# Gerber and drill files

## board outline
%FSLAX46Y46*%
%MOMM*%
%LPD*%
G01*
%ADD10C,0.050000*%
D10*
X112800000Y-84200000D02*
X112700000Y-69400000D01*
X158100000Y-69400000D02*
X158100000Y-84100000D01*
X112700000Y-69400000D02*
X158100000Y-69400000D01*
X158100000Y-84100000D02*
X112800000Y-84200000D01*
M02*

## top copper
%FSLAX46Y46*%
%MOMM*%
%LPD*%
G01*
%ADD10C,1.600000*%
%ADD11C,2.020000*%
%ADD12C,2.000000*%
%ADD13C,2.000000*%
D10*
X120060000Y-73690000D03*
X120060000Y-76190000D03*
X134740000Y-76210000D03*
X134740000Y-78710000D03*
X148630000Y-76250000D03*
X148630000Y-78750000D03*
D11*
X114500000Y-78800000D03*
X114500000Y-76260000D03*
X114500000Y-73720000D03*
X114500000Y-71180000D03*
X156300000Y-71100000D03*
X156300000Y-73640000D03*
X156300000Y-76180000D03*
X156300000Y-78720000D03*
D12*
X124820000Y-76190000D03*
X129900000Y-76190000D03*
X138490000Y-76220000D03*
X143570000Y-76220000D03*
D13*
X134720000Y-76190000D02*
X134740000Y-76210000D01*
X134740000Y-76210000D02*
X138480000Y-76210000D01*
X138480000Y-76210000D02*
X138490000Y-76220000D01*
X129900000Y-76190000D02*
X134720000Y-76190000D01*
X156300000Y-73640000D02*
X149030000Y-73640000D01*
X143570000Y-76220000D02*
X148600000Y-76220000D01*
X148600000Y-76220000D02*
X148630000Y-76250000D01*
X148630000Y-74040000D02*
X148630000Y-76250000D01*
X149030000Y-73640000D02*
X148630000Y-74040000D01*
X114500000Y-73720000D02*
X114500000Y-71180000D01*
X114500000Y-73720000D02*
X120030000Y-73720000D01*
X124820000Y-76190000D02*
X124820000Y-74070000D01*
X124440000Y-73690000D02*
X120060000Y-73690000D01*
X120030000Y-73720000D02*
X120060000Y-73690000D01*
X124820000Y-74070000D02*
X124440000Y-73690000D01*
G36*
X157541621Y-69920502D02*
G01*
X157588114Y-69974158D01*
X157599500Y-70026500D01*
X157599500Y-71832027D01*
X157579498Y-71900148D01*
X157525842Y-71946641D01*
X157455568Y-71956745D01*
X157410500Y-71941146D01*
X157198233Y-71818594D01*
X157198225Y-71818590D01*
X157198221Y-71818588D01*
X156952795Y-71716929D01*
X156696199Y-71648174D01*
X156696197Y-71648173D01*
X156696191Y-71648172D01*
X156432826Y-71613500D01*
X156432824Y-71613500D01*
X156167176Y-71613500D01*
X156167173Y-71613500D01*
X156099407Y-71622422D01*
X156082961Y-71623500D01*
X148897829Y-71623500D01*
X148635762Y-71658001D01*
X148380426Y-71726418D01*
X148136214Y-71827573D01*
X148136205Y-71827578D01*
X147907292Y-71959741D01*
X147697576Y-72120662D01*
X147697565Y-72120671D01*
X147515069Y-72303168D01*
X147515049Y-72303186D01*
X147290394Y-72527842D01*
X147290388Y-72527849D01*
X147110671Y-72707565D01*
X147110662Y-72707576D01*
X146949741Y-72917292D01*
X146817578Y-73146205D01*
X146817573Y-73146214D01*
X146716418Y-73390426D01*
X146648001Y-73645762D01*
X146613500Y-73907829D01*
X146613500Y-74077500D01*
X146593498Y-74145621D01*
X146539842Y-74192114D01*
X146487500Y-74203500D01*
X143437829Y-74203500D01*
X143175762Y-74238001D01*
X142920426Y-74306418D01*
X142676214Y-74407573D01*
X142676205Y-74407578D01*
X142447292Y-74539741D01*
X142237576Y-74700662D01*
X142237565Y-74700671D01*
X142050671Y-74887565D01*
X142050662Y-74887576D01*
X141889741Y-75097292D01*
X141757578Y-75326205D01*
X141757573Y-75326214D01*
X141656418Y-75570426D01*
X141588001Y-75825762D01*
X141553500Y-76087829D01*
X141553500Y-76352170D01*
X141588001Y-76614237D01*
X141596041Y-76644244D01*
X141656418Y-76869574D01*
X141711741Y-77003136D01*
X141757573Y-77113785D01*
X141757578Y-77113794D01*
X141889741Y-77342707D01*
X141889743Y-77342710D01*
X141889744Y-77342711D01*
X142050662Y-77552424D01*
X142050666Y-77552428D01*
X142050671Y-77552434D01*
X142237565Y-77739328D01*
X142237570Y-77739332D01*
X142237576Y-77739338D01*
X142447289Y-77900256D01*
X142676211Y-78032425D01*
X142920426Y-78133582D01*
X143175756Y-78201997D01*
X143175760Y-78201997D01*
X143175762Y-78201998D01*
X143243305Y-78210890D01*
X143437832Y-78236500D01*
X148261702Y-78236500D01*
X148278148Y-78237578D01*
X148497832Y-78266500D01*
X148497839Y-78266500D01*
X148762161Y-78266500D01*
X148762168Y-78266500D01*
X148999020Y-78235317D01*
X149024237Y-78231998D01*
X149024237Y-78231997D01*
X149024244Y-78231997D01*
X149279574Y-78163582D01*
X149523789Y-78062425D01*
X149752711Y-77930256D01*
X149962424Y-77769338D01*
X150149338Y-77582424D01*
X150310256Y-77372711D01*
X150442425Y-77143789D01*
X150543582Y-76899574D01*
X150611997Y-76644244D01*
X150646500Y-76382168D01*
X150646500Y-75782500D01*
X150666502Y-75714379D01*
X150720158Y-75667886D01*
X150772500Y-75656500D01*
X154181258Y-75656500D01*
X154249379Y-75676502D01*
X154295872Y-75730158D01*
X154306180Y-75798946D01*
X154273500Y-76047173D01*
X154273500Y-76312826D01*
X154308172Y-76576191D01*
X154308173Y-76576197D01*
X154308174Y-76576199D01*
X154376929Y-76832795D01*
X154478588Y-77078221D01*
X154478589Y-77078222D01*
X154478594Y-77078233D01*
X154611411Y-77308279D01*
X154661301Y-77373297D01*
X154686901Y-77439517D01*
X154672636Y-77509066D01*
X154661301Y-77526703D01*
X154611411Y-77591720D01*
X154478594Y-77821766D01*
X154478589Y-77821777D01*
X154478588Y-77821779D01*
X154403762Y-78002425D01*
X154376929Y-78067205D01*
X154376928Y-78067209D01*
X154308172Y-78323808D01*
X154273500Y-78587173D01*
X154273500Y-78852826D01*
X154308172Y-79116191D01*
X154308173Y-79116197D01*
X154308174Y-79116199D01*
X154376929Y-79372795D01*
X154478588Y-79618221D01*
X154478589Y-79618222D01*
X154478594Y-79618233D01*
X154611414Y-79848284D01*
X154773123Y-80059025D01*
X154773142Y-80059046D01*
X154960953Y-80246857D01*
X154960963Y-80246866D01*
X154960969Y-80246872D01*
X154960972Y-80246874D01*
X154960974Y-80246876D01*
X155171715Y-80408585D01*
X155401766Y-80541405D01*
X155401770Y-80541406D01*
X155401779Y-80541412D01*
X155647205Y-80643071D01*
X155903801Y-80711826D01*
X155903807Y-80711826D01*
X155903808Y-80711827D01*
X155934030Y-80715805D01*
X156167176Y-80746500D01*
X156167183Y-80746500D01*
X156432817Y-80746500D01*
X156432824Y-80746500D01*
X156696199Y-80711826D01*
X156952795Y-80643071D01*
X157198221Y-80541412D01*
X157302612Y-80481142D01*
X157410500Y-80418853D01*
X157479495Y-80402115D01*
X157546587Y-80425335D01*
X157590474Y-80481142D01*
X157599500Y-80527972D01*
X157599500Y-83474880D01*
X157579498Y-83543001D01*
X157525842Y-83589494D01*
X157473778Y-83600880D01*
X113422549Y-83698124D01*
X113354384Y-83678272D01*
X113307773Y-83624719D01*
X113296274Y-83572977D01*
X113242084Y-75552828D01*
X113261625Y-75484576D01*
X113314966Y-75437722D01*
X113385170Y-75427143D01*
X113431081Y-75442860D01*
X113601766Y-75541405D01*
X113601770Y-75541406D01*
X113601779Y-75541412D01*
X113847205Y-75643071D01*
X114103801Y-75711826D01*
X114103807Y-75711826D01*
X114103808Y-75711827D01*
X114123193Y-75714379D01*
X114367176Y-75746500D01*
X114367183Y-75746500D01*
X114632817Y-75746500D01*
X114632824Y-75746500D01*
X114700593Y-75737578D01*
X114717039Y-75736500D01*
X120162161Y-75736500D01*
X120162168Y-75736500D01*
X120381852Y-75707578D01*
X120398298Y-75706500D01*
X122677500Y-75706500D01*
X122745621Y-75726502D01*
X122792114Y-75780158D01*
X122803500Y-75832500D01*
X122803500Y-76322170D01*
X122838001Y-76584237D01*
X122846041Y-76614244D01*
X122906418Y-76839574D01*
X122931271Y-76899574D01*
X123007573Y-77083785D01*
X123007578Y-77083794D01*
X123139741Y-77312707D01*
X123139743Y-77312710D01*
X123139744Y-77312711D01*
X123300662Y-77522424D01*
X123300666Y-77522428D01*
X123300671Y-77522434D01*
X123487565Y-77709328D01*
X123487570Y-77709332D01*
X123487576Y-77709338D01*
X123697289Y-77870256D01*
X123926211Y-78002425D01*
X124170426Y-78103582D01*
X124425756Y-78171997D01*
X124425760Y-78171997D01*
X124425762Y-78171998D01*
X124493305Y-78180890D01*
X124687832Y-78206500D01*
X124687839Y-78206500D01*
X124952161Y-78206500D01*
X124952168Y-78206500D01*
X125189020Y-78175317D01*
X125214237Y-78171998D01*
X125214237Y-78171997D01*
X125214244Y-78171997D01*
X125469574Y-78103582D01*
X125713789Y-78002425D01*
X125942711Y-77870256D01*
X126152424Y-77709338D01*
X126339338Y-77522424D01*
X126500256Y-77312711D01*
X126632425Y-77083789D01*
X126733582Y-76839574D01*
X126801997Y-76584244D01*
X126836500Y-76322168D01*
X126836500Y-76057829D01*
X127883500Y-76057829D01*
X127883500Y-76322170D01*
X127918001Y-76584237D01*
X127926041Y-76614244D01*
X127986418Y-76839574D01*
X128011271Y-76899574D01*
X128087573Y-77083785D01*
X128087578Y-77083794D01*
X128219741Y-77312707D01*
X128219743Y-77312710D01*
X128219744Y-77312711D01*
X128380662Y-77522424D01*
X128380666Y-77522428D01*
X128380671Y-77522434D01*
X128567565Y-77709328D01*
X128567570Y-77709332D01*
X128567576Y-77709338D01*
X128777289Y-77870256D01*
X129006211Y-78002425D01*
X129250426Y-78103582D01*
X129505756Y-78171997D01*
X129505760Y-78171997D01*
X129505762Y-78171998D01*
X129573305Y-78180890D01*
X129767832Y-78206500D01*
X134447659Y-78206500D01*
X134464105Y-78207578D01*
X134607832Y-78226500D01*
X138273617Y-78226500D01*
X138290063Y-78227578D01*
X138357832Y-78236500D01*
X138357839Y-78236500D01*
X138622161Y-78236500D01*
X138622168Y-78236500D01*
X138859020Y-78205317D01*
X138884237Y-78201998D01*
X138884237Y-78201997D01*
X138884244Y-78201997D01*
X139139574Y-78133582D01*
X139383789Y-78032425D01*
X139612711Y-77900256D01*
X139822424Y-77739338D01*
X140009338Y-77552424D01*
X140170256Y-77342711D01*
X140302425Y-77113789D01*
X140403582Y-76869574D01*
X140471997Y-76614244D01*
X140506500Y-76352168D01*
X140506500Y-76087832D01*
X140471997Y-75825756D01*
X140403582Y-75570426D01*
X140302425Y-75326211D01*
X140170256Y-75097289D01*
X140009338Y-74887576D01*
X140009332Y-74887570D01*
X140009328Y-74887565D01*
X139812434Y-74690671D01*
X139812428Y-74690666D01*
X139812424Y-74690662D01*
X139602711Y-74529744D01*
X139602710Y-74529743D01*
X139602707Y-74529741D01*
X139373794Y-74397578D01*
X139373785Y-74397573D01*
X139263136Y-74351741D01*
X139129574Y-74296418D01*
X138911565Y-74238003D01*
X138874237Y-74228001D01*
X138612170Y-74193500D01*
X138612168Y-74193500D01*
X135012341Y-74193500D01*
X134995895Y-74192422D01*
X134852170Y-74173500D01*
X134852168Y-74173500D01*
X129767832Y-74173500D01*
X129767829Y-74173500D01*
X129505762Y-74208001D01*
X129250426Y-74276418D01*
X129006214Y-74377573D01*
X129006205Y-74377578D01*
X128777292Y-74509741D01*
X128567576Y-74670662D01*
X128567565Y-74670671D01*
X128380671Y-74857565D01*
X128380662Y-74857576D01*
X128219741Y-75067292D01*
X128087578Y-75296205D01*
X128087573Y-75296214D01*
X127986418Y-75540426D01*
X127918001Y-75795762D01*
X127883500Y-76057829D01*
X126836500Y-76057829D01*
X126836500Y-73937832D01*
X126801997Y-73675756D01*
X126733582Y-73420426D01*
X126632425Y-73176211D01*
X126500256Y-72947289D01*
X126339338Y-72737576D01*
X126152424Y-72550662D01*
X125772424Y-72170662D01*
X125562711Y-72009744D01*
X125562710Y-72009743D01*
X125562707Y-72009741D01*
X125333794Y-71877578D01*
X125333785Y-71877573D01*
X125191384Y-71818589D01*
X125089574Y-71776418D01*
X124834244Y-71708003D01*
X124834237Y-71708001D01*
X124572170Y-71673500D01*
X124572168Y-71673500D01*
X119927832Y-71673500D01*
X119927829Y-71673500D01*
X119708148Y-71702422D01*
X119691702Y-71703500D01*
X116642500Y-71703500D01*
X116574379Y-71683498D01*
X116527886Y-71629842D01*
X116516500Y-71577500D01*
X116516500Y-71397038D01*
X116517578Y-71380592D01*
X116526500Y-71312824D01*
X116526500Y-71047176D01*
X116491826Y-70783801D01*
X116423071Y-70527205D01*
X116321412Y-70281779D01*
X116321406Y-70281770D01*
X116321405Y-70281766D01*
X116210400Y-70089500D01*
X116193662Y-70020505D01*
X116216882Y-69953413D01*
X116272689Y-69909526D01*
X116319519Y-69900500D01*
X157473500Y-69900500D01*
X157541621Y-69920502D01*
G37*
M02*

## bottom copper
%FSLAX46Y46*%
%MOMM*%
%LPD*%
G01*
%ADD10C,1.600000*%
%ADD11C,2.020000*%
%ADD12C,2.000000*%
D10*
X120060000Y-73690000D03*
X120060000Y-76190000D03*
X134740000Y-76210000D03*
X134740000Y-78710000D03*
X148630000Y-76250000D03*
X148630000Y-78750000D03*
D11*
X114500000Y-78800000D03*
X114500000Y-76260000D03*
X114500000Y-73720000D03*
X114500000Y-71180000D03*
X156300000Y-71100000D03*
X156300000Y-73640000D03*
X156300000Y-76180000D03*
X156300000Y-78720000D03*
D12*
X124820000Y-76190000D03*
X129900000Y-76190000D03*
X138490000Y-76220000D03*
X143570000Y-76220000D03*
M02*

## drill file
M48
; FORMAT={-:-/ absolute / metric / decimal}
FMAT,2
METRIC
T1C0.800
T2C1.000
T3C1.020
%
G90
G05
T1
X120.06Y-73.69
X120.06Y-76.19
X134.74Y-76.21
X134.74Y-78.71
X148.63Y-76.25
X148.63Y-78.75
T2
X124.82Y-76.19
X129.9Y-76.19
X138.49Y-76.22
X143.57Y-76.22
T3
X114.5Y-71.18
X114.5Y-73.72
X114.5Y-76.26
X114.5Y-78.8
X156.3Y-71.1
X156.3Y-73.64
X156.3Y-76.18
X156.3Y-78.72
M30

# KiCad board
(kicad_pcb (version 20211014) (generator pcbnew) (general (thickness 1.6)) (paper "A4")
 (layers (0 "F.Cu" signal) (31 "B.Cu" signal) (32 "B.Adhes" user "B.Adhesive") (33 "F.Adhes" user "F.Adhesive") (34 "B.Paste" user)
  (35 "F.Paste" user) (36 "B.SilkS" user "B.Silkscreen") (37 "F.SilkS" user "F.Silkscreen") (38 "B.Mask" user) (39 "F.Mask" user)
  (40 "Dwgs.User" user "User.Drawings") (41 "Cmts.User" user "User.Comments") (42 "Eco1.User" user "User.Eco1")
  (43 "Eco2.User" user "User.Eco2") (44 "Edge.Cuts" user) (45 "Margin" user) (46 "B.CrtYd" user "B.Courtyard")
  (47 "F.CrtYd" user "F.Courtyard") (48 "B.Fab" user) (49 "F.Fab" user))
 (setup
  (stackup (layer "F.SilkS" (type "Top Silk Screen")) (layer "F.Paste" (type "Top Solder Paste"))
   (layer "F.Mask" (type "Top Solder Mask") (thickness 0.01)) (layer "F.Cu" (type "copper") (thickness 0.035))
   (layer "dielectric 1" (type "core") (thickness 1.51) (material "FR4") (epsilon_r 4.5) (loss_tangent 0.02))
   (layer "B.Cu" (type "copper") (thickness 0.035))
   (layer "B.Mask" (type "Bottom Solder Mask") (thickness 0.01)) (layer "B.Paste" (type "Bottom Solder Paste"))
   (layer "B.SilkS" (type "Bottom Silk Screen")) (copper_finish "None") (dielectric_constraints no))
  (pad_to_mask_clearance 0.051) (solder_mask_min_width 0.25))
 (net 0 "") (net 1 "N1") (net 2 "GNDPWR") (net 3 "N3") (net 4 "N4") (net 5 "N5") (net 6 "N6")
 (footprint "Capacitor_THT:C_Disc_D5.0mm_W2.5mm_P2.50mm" (layer "F.Cu") (at 120.06 73.69 -90)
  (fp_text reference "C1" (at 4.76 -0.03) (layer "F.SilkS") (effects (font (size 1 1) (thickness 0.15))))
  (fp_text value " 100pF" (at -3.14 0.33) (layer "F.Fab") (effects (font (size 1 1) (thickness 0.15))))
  (pad "1" thru_hole circle locked (at 0 0 270) (size 1.6 1.6) (drill 0.8) (layers *.Cu *.Mask) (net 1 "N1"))
  (pad "2" thru_hole circle locked (at 2.5 0 270) (size 1.6 1.6) (drill 0.8) (layers *.Cu *.Mask) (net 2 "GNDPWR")))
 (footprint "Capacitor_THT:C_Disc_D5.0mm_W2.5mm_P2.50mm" (layer "F.Cu") (at 134.74 76.21 -90)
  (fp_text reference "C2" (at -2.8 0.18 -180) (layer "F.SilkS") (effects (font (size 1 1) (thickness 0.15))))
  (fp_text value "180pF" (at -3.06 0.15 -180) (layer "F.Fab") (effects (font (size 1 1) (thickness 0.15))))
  (pad "1" thru_hole circle locked (at 0 0 270) (size 1.6 1.6) (drill 0.8) (layers *.Cu *.Mask) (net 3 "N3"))
  (pad "2" thru_hole circle locked (at 2.5 0 270) (size 1.6 1.6) (drill 0.8) (layers *.Cu *.Mask) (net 2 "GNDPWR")))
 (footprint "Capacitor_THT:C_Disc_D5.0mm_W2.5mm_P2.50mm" (layer "F.Cu") (at 148.63 76.25 -90)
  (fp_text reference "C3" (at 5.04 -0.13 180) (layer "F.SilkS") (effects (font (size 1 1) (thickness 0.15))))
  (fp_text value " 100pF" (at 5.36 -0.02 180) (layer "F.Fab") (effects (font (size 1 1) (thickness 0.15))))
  (pad "1" thru_hole circle locked (at 0 0 270) (size 1.6 1.6) (drill 0.8) (layers *.Cu *.Mask) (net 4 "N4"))
  (pad "2" thru_hole circle locked (at 2.5 0 270) (size 1.6 1.6) (drill 0.8) (layers *.Cu *.Mask) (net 2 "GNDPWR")))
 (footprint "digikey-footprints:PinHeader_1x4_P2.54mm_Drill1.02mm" (layer "F.Cu") (at 114.5 78.8 90)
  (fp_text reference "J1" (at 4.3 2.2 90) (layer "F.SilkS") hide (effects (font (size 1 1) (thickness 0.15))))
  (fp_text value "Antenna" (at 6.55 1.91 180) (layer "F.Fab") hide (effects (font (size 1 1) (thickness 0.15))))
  (pad "1" thru_hole circle locked (at 0 0 90) (size 2.02 2.02) (drill 1.02) (layers *.Cu *.Mask) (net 2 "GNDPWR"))
  (pad "2" thru_hole circle locked (at 2.54 0 90) (size 2.02 2.02) (drill 1.02) (layers *.Cu *.Mask) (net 2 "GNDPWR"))
  (pad "3" thru_hole circle locked (at 5.08 0 90) (size 2.02 2.02) (drill 1.02) (layers *.Cu *.Mask) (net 1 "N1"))
  (pad "4" thru_hole circle locked (at 7.62 0 90) (size 2.02 2.02) (drill 1.02) (layers *.Cu *.Mask) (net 1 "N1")))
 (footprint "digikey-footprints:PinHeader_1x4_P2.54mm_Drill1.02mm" (layer "F.Cu") (at 156.3 71.1 -90)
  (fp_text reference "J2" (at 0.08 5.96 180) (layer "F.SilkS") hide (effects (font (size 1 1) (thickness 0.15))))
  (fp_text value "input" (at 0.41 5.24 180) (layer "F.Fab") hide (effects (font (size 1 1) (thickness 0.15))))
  (pad "1" thru_hole circle locked (at 0 0 270) (size 2.02 2.02) (drill 1.02) (layers *.Cu *.Mask) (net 2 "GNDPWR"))
  (pad "2" thru_hole circle locked (at 2.54 0 270) (size 2.02 2.02) (drill 1.02) (layers *.Cu *.Mask) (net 4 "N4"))
  (pad "3" thru_hole circle locked (at 5.08 0 270) (size 2.02 2.02) (drill 1.02) (layers *.Cu *.Mask) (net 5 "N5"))
  (pad "4" thru_hole circle locked (at 7.62 0 270) (size 2.02 2.02) (drill 1.02) (layers *.Cu *.Mask) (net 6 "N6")))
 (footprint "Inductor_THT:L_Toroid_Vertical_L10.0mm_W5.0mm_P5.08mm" (layer "F.Cu") (at 124.82 76.19 90)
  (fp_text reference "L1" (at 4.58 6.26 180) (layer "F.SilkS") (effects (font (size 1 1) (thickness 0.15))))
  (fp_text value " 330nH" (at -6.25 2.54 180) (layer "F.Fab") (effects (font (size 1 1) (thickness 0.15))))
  (pad "1" thru_hole circle locked (at 0 0 90) (size 2 2) (drill 1) (layers *.Cu *.Mask) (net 1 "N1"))
  (pad "2" thru_hole circle locked (at 0 5.08 90) (size 2 2) (drill 1) (layers *.Cu *.Mask) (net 3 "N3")))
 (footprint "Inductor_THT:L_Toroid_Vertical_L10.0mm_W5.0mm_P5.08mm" (layer "F.Cu") (at 138.49 76.22 90)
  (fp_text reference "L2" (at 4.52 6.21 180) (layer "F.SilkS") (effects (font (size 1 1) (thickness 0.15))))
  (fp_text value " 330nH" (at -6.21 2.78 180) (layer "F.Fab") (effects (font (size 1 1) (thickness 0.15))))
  (pad "1" thru_hole circle locked (at 0 0 90) (size 2 2) (drill 1) (layers *.Cu *.Mask) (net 3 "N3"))
  (pad "2" thru_hole circle locked (at 0 5.08 90) (size 2 2) (drill 1) (layers *.Cu *.Mask) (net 4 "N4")))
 (gr_line (start 112.8 84.2) (end 112.7 69.4) (layer "Edge.Cuts") (width 0.05))
 (gr_line (start 158.1 69.4) (end 158.1 84.1) (layer "Edge.Cuts") (width 0.05))
 (gr_line (start 112.7 69.4) (end 158.1 69.4) (layer "Edge.Cuts") (width 0.05))
 (gr_line (start 158.1 84.1) (end 112.8 84.2) (layer "Edge.Cuts") (width 0.05))
 (segment (start 134.72 76.19) (end 134.74 76.21) (width 2) (layer "F.Cu") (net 3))
 (segment (start 134.74 76.21) (end 138.48 76.21) (width 2) (layer "F.Cu") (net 3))
 (segment (start 138.48 76.21) (end 138.49 76.22) (width 2) (layer "F.Cu") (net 3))
 (segment (start 129.9 76.19) (end 134.72 76.19) (width 2) (layer "F.Cu") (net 3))
 (segment (start 156.3 73.64) (end 149.03 73.64) (width 2) (layer "F.Cu") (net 4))
 (segment (start 143.57 76.22) (end 148.6 76.22) (width 2) (layer "F.Cu") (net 4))
 (segment (start 148.6 76.22) (end 148.63 76.25) (width 2) (layer "F.Cu") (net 4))
 (segment (start 148.63 74.04) (end 148.63 76.25) (width 2) (layer "F.Cu") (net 4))
 (segment (start 149.03 73.64) (end 148.63 74.04) (width 2) (layer "F.Cu") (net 4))
 (segment (start 114.5 73.72) (end 114.5 71.18) (width 2) (layer "F.Cu") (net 1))
 (segment (start 114.5 73.72) (end 120.03 73.72) (width 2) (layer "F.Cu") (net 1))
 (segment (start 124.82 76.19) (end 124.82 74.07) (width 2) (layer "F.Cu") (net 1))
 (segment (start 124.44 73.69) (end 120.06 73.69) (width 2) (layer "F.Cu") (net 1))
 (segment (start 120.03 73.72) (end 120.06 73.69) (width 2) (layer "F.Cu") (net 1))
 (segment (start 124.82 74.07) (end 124.44 73.69) (width 2) (layer "F.Cu") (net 1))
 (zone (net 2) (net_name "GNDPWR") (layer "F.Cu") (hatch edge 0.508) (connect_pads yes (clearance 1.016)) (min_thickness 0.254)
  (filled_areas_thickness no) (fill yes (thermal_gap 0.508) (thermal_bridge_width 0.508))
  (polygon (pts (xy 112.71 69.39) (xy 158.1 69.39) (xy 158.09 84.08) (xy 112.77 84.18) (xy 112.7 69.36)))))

